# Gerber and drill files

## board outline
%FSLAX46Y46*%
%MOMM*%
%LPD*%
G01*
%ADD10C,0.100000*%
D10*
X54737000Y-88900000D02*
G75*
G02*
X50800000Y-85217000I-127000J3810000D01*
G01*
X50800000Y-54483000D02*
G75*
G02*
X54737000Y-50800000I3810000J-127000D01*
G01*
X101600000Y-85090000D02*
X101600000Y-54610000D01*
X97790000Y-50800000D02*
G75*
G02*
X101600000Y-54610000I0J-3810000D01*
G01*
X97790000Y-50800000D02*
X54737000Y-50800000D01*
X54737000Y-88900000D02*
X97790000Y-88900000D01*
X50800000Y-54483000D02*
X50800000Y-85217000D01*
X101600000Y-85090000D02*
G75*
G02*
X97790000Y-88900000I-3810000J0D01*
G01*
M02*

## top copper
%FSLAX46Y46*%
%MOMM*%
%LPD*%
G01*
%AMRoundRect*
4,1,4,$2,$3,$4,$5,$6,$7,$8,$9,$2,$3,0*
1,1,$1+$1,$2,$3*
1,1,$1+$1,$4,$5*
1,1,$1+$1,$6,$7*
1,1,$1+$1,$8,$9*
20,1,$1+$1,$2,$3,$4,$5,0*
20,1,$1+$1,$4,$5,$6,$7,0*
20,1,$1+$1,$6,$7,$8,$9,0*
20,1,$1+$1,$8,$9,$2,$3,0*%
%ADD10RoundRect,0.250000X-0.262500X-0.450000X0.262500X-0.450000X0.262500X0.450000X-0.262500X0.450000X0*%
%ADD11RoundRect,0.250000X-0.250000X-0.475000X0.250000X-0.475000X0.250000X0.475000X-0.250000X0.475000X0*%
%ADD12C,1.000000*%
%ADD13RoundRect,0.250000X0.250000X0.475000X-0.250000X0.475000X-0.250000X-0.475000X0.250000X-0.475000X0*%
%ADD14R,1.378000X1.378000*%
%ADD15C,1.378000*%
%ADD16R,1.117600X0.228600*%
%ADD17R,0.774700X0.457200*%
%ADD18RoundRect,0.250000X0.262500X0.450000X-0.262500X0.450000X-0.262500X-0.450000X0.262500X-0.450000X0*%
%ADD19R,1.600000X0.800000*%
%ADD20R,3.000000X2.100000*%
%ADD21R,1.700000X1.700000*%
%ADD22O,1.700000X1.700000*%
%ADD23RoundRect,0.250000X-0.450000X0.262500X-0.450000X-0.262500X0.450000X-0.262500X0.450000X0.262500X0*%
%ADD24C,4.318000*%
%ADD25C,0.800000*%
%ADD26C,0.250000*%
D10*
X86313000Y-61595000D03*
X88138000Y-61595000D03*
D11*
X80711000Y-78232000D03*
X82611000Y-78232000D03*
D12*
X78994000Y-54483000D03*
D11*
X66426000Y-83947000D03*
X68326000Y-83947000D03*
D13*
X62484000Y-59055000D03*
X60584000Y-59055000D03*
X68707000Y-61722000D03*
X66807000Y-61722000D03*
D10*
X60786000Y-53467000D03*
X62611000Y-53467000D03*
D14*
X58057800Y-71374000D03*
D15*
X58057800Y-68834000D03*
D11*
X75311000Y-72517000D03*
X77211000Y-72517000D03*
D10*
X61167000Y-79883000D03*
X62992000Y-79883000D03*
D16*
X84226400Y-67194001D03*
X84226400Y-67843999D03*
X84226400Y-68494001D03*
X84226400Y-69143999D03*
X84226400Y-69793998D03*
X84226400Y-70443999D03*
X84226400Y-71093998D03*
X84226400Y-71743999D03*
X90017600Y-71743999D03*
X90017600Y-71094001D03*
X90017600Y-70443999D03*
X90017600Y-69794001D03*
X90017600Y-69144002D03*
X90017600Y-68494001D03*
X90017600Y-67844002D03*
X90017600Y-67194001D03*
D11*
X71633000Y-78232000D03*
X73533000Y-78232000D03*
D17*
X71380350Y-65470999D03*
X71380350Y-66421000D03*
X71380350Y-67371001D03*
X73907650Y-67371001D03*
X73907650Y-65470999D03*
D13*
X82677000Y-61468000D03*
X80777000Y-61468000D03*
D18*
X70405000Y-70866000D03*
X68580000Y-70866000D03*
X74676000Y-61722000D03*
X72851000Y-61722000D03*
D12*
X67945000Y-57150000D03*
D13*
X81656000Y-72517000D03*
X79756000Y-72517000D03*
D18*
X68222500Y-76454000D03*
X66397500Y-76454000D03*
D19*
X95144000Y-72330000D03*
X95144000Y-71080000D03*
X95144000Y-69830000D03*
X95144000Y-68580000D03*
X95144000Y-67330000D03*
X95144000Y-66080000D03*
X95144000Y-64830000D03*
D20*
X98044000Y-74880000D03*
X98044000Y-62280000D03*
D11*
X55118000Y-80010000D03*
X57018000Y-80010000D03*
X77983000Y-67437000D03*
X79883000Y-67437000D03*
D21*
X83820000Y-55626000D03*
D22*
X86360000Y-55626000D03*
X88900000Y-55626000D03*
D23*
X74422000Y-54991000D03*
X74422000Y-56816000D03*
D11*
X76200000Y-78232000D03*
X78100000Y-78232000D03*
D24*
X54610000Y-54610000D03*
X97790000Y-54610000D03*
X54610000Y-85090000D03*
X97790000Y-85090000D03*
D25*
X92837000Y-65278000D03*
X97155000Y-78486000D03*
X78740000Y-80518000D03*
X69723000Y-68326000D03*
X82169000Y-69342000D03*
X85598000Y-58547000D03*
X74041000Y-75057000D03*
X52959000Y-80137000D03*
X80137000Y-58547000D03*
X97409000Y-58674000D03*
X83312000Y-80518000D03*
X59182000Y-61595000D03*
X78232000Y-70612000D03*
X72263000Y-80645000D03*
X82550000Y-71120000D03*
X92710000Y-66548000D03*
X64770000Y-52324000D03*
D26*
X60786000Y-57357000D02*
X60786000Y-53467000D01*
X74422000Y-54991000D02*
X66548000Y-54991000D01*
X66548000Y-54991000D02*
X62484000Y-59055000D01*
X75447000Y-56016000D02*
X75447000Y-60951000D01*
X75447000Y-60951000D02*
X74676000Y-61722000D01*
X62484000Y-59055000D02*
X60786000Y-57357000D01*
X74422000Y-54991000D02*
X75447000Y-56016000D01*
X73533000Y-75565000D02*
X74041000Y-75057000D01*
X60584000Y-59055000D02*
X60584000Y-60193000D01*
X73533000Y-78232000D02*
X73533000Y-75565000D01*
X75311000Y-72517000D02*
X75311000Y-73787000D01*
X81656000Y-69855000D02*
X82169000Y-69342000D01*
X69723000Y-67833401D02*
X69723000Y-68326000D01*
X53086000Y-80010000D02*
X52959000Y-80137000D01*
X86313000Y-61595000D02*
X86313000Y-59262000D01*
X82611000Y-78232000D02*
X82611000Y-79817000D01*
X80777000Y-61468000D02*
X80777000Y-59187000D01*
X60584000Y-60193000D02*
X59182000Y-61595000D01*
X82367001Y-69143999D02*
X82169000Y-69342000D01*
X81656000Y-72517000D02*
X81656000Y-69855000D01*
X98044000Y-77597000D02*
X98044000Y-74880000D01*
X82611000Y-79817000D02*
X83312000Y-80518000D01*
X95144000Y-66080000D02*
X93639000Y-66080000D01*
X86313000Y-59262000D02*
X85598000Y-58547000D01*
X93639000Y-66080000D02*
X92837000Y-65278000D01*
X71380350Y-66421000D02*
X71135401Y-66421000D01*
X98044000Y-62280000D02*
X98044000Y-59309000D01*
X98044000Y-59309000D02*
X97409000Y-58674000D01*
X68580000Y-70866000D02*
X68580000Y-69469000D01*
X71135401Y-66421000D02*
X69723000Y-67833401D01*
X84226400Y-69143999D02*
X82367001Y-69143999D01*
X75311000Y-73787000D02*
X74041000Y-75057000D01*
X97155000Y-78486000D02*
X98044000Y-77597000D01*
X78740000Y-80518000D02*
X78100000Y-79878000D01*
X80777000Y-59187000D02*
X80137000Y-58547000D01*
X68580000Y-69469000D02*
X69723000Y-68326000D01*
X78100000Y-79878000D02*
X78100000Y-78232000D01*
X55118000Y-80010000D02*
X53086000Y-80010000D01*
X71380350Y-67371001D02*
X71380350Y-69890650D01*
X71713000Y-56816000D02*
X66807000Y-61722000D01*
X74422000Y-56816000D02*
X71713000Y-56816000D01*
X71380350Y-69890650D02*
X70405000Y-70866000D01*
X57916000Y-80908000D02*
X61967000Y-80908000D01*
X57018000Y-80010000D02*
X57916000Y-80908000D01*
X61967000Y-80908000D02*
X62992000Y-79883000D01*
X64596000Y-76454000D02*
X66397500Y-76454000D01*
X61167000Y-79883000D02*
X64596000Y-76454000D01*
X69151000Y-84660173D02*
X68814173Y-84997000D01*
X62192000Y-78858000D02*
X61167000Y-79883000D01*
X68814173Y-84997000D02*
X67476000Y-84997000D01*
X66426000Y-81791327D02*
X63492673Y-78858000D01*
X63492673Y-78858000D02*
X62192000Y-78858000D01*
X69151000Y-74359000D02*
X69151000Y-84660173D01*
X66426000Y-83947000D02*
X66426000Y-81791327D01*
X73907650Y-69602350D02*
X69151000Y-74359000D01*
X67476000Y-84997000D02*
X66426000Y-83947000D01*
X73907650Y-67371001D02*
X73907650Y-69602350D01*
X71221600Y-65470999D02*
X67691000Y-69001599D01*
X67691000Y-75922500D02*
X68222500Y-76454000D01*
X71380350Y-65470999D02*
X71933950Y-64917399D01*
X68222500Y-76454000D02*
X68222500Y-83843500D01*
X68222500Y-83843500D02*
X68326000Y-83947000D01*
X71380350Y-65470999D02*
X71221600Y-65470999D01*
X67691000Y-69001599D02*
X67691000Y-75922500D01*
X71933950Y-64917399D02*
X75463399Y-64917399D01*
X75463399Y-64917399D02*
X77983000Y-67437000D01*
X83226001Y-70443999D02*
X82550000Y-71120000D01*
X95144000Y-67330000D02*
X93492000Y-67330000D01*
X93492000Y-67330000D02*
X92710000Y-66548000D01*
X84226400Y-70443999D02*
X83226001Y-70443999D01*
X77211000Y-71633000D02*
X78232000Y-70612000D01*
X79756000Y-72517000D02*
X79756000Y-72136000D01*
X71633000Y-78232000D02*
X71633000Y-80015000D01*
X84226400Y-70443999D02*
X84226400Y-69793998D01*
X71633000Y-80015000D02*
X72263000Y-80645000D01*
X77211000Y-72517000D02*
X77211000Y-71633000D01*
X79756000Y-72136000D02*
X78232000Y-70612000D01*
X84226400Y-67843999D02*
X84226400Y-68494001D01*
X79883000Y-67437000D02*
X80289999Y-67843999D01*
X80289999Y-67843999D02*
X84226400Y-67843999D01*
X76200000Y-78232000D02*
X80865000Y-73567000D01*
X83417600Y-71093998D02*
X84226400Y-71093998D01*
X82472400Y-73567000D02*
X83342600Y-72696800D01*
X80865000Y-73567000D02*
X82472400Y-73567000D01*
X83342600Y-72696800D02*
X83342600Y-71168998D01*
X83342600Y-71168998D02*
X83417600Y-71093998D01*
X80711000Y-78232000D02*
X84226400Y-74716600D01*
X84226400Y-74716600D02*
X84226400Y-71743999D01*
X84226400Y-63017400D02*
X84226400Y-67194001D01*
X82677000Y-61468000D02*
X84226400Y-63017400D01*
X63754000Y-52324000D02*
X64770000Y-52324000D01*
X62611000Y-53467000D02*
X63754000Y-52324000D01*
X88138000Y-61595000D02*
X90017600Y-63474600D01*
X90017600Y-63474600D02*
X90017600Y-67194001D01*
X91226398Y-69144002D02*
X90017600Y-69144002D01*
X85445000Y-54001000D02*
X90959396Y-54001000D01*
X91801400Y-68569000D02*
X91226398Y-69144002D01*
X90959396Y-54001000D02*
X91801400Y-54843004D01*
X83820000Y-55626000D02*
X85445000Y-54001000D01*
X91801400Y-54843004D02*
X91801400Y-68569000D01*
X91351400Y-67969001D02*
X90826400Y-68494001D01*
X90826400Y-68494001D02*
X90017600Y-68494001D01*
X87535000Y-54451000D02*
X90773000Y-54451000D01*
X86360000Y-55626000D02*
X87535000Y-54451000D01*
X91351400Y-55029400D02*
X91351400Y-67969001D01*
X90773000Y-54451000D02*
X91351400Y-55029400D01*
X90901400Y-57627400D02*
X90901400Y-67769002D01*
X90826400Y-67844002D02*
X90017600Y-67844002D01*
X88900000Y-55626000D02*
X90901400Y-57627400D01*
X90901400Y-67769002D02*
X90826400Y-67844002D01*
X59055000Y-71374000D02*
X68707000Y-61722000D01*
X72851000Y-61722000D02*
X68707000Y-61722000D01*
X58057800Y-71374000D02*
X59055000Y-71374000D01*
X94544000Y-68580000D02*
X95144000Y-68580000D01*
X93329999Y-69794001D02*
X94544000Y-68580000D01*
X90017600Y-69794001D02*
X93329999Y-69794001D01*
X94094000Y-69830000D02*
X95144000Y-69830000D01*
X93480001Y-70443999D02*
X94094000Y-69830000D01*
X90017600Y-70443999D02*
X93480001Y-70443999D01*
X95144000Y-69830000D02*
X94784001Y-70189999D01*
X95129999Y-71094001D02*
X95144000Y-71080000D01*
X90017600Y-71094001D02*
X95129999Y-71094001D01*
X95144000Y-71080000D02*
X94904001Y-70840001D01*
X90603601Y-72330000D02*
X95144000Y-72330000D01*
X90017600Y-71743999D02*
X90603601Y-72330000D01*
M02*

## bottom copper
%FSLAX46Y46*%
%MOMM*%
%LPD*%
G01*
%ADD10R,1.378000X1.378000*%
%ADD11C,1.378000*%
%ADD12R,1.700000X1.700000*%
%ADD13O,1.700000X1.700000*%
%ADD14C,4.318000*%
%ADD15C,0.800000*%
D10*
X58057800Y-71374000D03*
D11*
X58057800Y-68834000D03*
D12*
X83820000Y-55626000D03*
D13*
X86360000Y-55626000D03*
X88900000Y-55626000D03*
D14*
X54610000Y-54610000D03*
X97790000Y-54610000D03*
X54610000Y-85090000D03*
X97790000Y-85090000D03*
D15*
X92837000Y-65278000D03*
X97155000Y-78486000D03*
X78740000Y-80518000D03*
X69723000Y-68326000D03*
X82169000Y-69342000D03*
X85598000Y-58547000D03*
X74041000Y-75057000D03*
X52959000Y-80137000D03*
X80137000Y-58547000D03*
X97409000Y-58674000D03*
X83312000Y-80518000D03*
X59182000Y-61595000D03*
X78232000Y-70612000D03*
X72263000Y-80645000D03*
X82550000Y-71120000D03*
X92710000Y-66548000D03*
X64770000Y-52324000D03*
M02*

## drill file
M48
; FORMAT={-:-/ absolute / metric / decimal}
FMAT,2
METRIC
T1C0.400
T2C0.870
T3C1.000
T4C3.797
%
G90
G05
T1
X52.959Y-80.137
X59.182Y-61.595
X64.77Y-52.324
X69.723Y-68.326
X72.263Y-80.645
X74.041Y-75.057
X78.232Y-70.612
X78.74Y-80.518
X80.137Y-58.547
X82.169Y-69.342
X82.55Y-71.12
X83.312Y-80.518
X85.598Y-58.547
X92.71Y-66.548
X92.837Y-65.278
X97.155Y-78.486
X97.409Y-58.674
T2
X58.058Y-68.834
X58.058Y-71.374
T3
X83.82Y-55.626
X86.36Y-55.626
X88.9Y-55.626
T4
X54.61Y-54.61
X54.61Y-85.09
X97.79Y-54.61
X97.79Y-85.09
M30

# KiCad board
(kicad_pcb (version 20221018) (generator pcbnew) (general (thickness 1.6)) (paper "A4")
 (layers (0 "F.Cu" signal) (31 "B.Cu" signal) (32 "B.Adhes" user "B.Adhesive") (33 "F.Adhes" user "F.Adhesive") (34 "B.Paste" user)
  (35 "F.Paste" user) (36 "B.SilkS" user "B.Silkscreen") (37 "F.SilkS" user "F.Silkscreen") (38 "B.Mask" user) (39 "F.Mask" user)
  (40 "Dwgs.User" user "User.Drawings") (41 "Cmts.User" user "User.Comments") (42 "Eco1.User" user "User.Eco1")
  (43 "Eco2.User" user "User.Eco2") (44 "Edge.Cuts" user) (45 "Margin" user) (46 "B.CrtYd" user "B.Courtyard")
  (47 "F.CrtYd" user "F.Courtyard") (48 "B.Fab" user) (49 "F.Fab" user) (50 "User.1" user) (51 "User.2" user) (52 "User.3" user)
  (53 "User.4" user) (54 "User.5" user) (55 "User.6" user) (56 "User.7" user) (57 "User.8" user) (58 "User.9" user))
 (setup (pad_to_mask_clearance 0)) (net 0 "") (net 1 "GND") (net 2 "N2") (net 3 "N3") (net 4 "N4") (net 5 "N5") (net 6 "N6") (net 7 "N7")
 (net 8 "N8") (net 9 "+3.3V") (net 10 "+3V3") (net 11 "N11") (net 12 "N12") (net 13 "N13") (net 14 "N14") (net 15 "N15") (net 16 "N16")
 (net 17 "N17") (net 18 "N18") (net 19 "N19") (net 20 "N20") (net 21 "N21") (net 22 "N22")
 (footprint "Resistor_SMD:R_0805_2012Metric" (layer "F.Cu") (at 87.2255 61.595)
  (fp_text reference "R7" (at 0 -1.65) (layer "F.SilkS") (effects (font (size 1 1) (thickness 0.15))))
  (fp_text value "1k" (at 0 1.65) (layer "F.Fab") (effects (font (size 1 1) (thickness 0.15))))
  (pad "1" smd roundrect (at -0.9125 0) (size 1.025 1.4) (layers "F.Cu" "F.Paste" "F.Mask") (roundrect_rratio 0.243902) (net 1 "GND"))
  (pad "2" smd roundrect (at 0.9125 0) (size 1.025 1.4) (layers "F.Cu" "F.Paste" "F.Mask") (roundrect_rratio 0.243902) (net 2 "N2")))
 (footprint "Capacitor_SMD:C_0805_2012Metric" (layer "F.Cu") (at 81.661 78.232)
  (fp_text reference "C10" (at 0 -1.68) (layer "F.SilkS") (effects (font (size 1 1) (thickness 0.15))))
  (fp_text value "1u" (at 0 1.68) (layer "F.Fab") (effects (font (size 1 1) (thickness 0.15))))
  (pad "1" smd roundrect (at -0.95 0) (size 1 1.45) (layers "F.Cu" "F.Paste" "F.Mask") (roundrect_rratio 0.25) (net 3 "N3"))
  (pad "2" smd roundrect (at 0.95 0) (size 1 1.45) (layers "F.Cu" "F.Paste" "F.Mask") (roundrect_rratio 0.25) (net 1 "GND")))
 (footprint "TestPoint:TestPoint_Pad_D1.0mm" (layer "F.Cu") (at 78.994 54.483)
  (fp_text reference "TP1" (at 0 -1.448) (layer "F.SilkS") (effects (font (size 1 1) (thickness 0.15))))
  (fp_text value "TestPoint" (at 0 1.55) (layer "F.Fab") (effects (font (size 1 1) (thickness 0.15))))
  (pad "1" smd circle (at 0 0) (size 1 1) (layers "F.Cu" "F.Mask") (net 1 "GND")))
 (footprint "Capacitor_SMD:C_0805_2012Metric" (layer "F.Cu") (at 67.376 83.947)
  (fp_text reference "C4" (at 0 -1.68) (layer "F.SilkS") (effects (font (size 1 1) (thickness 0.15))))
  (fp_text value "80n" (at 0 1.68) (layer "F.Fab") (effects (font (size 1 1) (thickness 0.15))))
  (pad "1" smd roundrect (at -0.95 0) (size 1 1.45) (layers "F.Cu" "F.Paste" "F.Mask") (roundrect_rratio 0.25) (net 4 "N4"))
  (pad "2" smd roundrect (at 0.95 0) (size 1 1.45) (layers "F.Cu" "F.Paste" "F.Mask") (roundrect_rratio 0.25) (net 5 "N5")))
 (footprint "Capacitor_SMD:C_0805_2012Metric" (layer "F.Cu") (at 61.534 59.055 180)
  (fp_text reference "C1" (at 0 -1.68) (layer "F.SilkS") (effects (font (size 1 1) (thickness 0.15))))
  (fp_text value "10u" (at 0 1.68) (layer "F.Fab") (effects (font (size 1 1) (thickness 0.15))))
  (pad "1" smd roundrect (at -0.95 0 180) (size 1 1.45) (layers "F.Cu" "F.Paste" "F.Mask") (roundrect_rratio 0.25) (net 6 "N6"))
  (pad "2" smd roundrect (at 0.95 0 180) (size 1 1.45) (layers "F.Cu" "F.Paste" "F.Mask") (roundrect_rratio 0.25) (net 1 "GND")))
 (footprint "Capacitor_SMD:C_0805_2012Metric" (layer "F.Cu") (at 67.757 61.722 180)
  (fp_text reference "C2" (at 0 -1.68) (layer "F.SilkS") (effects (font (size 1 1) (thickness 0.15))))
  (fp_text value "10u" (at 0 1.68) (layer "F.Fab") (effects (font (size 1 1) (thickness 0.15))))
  (pad "1" smd roundrect (at -0.95 0 180) (size 1 1.45) (layers "F.Cu" "F.Paste" "F.Mask") (roundrect_rratio 0.25) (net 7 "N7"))
  (pad "2" smd roundrect (at 0.95 0 180) (size 1 1.45) (layers "F.Cu" "F.Paste" "F.Mask") (roundrect_rratio 0.25) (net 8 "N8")))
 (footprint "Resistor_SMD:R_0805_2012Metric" (layer "F.Cu") (at 61.6985 53.467)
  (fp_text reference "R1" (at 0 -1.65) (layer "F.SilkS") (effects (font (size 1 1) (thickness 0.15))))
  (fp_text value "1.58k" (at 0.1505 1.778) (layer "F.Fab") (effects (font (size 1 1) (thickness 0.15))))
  (pad "1" smd roundrect (at -0.9125 0) (size 1.025 1.4) (layers "F.Cu" "F.Paste" "F.Mask") (roundrect_rratio 0.243902) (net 6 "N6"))
  (pad "2" smd roundrect (at 0.9125 0) (size 1.025 1.4) (layers "F.Cu" "F.Paste" "F.Mask") (roundrect_rratio 0.243902) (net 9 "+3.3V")))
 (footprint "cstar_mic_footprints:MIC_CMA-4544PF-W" (layer "F.Cu") (at 56.0578 70.104)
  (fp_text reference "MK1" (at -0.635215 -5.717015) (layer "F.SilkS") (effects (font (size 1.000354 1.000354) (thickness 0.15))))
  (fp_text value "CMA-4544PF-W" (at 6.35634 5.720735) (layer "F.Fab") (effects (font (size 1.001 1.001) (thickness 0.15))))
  (pad "1" thru_hole rect (at 2 1.27) (size 1.378 1.378) (drill 0.87) (layers "*.Cu" "*.Mask") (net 7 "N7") (solder_mask_margin 0.102))
  (pad "2" thru_hole circle (at 2 -1.27) (size 1.378 1.378) (drill 0.87) (layers "*.Cu" "*.Mask") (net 1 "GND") (solder_mask_margin 0.102)))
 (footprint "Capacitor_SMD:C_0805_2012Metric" (layer "F.Cu") (at 76.261 72.517)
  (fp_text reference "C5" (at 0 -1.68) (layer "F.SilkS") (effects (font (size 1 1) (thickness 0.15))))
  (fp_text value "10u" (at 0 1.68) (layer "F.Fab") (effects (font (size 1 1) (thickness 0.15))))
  (pad "1" smd roundrect (at -0.95 0) (size 1 1.45) (layers "F.Cu" "F.Paste" "F.Mask") (roundrect_rratio 0.25) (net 1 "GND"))
  (pad "2" smd roundrect (at 0.95 0) (size 1 1.45) (layers "F.Cu" "F.Paste" "F.Mask") (roundrect_rratio 0.25) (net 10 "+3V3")))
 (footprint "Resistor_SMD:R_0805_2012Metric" (layer "F.Cu") (at 62.0795 79.883)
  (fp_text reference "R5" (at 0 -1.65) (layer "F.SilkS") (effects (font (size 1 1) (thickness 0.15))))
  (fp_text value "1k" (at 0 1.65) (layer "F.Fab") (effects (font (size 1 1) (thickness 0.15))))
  (pad "1" smd roundrect (at -0.9125 0) (size 1.025 1.4) (layers "F.Cu" "F.Paste" "F.Mask") (roundrect_rratio 0.243902) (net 4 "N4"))
  (pad "2" smd roundrect (at 0.9125 0) (size 1.025 1.4) (layers "F.Cu" "F.Paste" "F.Mask") (roundrect_rratio 0.243902) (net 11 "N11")))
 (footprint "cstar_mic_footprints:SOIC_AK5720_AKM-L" (layer "F.Cu") (at 87.122 69.469)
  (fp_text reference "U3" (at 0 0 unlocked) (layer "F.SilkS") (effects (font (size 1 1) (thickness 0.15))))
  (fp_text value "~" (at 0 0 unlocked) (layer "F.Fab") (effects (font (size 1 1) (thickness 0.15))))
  (pad "1" smd rect (at -2.8956 -2.274999) (size 1.1176 0.2286) (layers "F.Cu" "F.Paste" "F.Mask") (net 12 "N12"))
  (pad "2" smd rect (at -2.8956 -1.625001) (size 1.1176 0.2286) (layers "F.Cu" "F.Paste" "F.Mask") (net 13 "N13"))
  (pad "3" smd rect (at -2.8956 -0.974999) (size 1.1176 0.2286) (layers "F.Cu" "F.Paste" "F.Mask") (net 13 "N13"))
  (pad "4" smd rect (at -2.8956 -0.325001) (size 1.1176 0.2286) (layers "F.Cu" "F.Paste" "F.Mask") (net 1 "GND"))
  (pad "5" smd rect (at -2.8956 0.324998) (size 1.1176 0.2286) (layers "F.Cu" "F.Paste" "F.Mask") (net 10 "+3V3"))
  (pad "6" smd rect (at -2.8956 0.974999) (size 1.1176 0.2286) (layers "F.Cu" "F.Paste" "F.Mask") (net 10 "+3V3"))
  (pad "7" smd rect (at -2.8956 1.624998) (size 1.1176 0.2286) (layers "F.Cu" "F.Paste" "F.Mask") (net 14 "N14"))
  (pad "8" smd rect (at -2.8956 2.274999) (size 1.1176 0.2286) (layers "F.Cu" "F.Paste" "F.Mask") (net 3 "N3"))
  (pad "9" smd rect (at 2.8956 2.274999) (size 1.1176 0.2286) (layers "F.Cu" "F.Paste" "F.Mask") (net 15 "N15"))
  (pad "10" smd rect (at 2.8956 1.625001) (size 1.1176 0.2286) (layers "F.Cu" "F.Paste" "F.Mask") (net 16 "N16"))
  (pad "11" smd rect (at 2.8956 0.974999) (size 1.1176 0.2286) (layers "F.Cu" "F.Paste" "F.Mask") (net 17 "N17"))
  (pad "12" smd rect (at 2.8956 0.325001) (size 1.1176 0.2286) (layers "F.Cu" "F.Paste" "F.Mask") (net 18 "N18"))
  (pad "13" smd rect (at 2.8956 -0.324998) (size 1.1176 0.2286) (layers "F.Cu" "F.Paste" "F.Mask") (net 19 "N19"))
  (pad "14" smd rect (at 2.8956 -0.974999) (size 1.1176 0.2286) (layers "F.Cu" "F.Paste" "F.Mask") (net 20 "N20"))
  (pad "15" smd rect (at 2.8956 -1.624998) (size 1.1176 0.2286) (layers "F.Cu" "F.Paste" "F.Mask") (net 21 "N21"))
  (pad "16" smd rect (at 2.8956 -2.274999) (size 1.1176 0.2286) (layers "F.Cu" "F.Paste" "F.Mask") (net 2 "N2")))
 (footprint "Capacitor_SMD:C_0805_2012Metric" (layer "F.Cu") (at 72.583 78.232)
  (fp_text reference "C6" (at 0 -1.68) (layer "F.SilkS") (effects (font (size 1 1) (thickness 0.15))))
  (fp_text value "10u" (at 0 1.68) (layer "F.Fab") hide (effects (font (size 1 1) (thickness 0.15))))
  (pad "1" smd roundrect (at -0.95 0) (size 1 1.45) (layers "F.Cu" "F.Paste" "F.Mask") (roundrect_rratio 0.25) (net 10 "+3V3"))
  (pad "2" smd roundrect (at 0.95 0) (size 1 1.45) (layers "F.Cu" "F.Paste" "F.Mask") (roundrect_rratio 0.25) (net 1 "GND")))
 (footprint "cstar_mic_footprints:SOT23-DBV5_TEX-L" (layer "F.Cu") (at 72.644 66.421)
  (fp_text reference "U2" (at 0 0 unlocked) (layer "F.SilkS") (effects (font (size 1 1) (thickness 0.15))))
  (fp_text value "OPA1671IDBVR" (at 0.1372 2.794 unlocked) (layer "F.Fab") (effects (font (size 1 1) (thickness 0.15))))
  (pad "1" smd rect (at -1.26365 -0.950001) (size 0.7747 0.4572) (layers "F.Cu" "F.Paste" "F.Mask") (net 5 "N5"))
  (pad "2" smd rect (at -1.26365 0) (size 0.7747 0.4572) (layers "F.Cu" "F.Paste" "F.Mask") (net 1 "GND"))
  (pad "3" smd rect (at -1.26365 0.950001) (size 0.7747 0.4572) (layers "F.Cu" "F.Paste" "F.Mask") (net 8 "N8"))
  (pad "4" smd rect (at 1.26365 0.950001) (size 0.7747 0.4572) (layers "F.Cu" "F.Paste" "F.Mask") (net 4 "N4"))
  (pad "5" smd rect (at 1.26365 -0.950001) (size 0.7747 0.4572) (layers "F.Cu" "F.Paste" "F.Mask") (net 9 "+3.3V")))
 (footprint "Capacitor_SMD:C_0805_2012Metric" (layer "F.Cu") (at 81.727 61.468 180)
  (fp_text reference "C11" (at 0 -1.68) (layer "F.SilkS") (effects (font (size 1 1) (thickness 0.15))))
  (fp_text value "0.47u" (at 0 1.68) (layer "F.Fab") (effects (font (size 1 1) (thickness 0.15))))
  (pad "1" smd roundrect (at -0.95 0 180) (size 1 1.45) (layers "F.Cu" "F.Paste" "F.Mask") (roundrect_rratio 0.25) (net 12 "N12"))
  (pad "2" smd roundrect (at 0.95 0 180) (size 1 1.45) (layers "F.Cu" "F.Paste" "F.Mask") (roundrect_rratio 0.25) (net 1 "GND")))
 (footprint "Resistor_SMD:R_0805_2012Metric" (layer "F.Cu") (at 69.4925 70.866 180)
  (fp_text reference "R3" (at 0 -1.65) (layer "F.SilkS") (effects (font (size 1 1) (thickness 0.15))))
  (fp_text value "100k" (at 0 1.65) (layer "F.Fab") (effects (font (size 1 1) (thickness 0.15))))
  (pad "1" smd roundrect (at -0.9125 0 180) (size 1.025 1.4) (layers "F.Cu" "F.Paste" "F.Mask") (roundrect_rratio 0.243902) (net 8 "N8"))
  (pad "2" smd roundrect (at 0.9125 0 180) (size 1.025 1.4) (layers "F.Cu" "F.Paste" "F.Mask") (roundrect_rratio 0.243902) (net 1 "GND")))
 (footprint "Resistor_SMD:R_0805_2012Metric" (layer "F.Cu") (at 73.7635 61.722 180)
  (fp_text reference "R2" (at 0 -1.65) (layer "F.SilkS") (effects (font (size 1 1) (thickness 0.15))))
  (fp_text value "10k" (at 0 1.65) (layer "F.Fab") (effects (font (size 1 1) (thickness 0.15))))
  (pad "1" smd roundrect (at -0.9125 0 180) (size 1.025 1.4) (layers "F.Cu" "F.Paste" "F.Mask") (roundrect_rratio 0.243902) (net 6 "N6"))
  (pad "2" smd roundrect (at 0.9125 0 180) (size 1.025 1.4) (layers "F.Cu" "F.Paste" "F.Mask") (roundrect_rratio 0.243902) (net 7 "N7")))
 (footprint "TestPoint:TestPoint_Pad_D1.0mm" (layer "F.Cu") (at 67.945 57.15)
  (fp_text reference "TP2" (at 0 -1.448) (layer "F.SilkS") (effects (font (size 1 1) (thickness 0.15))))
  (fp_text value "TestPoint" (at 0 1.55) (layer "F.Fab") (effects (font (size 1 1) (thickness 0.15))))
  (pad "1" smd circle (at 0 0) (size 1 1) (layers "F.Cu" "F.Mask") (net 8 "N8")))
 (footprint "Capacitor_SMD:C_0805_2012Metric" (layer "F.Cu") (at 80.706 72.517 180)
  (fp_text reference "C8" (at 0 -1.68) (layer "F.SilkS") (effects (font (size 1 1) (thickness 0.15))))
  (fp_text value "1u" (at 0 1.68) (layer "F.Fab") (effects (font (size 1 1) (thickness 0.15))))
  (pad "1" smd roundrect (at -0.95 0 180) (size 1 1.45) (layers "F.Cu" "F.Paste" "F.Mask") (roundrect_rratio 0.25) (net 1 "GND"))
  (pad "2" smd roundrect (at 0.95 0 180) (size 1 1.45) (layers "F.Cu" "F.Paste" "F.Mask") (roundrect_rratio 0.25) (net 10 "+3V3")))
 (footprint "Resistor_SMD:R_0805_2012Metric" (layer "F.Cu") (at 67.31 76.454 180)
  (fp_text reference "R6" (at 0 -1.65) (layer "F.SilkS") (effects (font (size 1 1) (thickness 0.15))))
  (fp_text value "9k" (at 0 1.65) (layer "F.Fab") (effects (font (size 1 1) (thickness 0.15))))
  (pad "1" smd roundrect (at -0.9125 0 180) (size 1.025 1.4) (layers "F.Cu" "F.Paste" "F.Mask") (roundrect_rratio 0.243902) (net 5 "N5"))
  (pad "2" smd roundrect (at 0.9125 0 180) (size 1.025 1.4) (layers "F.Cu" "F.Paste" "F.Mask") (roundrect_rratio 0.243902) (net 4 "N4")))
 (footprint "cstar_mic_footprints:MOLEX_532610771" (layer "F.Cu") (at 97.544 68.58 90)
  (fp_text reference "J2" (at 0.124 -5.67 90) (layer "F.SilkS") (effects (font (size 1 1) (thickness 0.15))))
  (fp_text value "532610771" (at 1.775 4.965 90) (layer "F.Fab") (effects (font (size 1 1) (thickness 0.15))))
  (pad "1" smd rect (at -3.75 -2.4 90) (size 0.8 1.6) (layers "F.Cu" "F.Paste") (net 15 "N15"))
  (pad "2" smd rect (at -2.5 -2.4 90) (size 0.8 1.6) (layers "F.Cu" "F.Paste") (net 16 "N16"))
  (pad "3" smd rect (at -1.25 -2.4 90) (size 0.8 1.6) (layers "F.Cu" "F.Paste") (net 17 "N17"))
  (pad "4" smd rect (at 0 -2.4 90) (size 0.8 1.6) (layers "F.Cu" "F.Paste") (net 18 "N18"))
  (pad "5" smd rect (at 1.25 -2.4 90) (size 0.8 1.6) (layers "F.Cu" "F.Paste") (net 10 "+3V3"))
  (pad "6" smd rect (at 2.5 -2.4 90) (size 0.8 1.6) (layers "F.Cu" "F.Paste") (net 1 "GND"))
  (pad "7" smd rect (at 3.75 -2.4 90) (size 0.8 1.6) (layers "F.Cu" "F.Paste") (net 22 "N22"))
  (pad "S1" smd rect (at -6.3 0.5 90) (size 2.1 3) (layers "F.Cu" "F.Paste") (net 1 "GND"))
  (pad "S2" smd rect (at 6.3 0.5 90) (size 2.1 3) (layers "F.Cu" "F.Paste") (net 1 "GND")))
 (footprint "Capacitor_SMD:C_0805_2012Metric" (layer "F.Cu") (at 56.068 80.01)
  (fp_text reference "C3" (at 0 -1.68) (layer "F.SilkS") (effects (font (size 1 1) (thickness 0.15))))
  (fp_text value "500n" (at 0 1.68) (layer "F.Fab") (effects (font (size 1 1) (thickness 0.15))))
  (pad "1" smd roundrect (at -0.95 0) (size 1 1.45) (layers "F.Cu" "F.Paste" "F.Mask") (roundrect_rratio 0.25) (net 1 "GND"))
  (pad "2" smd roundrect (at 0.95 0) (size 1 1.45) (layers "F.Cu" "F.Paste" "F.Mask") (roundrect_rratio 0.25) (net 11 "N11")))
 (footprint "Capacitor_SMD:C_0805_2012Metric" (layer "F.Cu") (at 78.933 67.437)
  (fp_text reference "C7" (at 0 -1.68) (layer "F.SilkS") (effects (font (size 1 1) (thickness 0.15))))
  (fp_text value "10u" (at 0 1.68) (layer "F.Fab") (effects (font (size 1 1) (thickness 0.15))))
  (pad "1" smd roundrect (at -0.95 0) (size 1 1.45) (layers "F.Cu" "F.Paste" "F.Mask") (roundrect_rratio 0.25) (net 5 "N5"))
  (pad "2" smd roundrect (at 0.95 0) (size 1 1.45) (layers "F.Cu" "F.Paste" "F.Mask") (roundrect_rratio 0.25) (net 13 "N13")))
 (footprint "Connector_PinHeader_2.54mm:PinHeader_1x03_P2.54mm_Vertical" (layer "F.Cu") (at 83.82 55.626 90)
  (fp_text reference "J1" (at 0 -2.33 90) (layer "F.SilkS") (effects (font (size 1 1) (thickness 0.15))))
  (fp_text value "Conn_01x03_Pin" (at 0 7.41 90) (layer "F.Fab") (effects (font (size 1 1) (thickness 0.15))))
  (pad "1" thru_hole rect (at 0 0 90) (size 1.7 1.7) (drill 1) (layers "*.Cu" "*.Mask") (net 19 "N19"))
  (pad "2" thru_hole oval (at 0 2.54 90) (size 1.7 1.7) (drill 1) (layers "*.Cu" "*.Mask") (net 20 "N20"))
  (pad "3" thru_hole oval (at 0 5.08 90) (size 1.7 1.7) (drill 1) (layers "*.Cu" "*.Mask") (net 21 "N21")))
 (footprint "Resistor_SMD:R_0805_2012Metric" (layer "F.Cu") (at 74.422 55.9035 -90)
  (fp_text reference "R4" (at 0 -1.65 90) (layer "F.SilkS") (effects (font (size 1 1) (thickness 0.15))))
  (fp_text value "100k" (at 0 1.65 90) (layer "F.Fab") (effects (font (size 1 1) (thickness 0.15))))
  (pad "1" smd roundrect (at -0.9125 0 270) (size 1.025 1.4) (layers "F.Cu" "F.Paste" "F.Mask") (roundrect_rratio 0.243902) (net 6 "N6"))
  (pad "2" smd roundrect (at 0.9125 0 270) (size 1.025 1.4) (layers "F.Cu" "F.Paste" "F.Mask") (roundrect_rratio 0.243902) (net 8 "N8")))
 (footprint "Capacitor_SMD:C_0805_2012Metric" (layer "F.Cu") (at 77.15 78.232)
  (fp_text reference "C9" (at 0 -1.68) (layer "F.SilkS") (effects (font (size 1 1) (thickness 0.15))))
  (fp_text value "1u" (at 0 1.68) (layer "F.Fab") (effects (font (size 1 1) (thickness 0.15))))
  (pad "1" smd roundrect (at -0.95 0) (size 1 1.45) (layers "F.Cu" "F.Paste" "F.Mask") (roundrect_rratio 0.25) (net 14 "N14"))
  (pad "2" smd roundrect (at 0.95 0) (size 1 1.45) (layers "F.Cu" "F.Paste" "F.Mask") (roundrect_rratio 0.25) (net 1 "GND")))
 (gr_arc (start 54.737 88.9) (mid 52.005726 87.873879) (end 50.8 85.217) (stroke (width 0.1) (type default)) (layer "Edge.Cuts"))
 (gr_arc (start 50.8 54.483) (mid 52.005726 51.826121) (end 54.737 50.8) (stroke (width 0.1) (type default)) (layer "Edge.Cuts"))
 (gr_line (start 101.6 85.09) (end 101.6 54.61) (stroke (width 0.1) (type default)) (layer "Edge.Cuts"))
 (gr_arc (start 97.79 50.8) (mid 100.484076 51.915923) (end 101.6 54.61) (stroke (width 0.1) (type default)) (layer "Edge.Cuts"))
 (gr_line (start 97.79 50.8) (end 54.737 50.8) (stroke (width 0.1) (type default)) (layer "Edge.Cuts"))
 (gr_line (start 54.737 88.9) (end 97.79 88.9) (stroke (width 0.1) (type default)) (layer "Edge.Cuts"))
 (gr_line (start 50.8 54.483) (end 50.8 85.217) (stroke (width 0.1) (type default)) (layer "Edge.Cuts"))
 (gr_arc (start 101.6 85.09) (mid 100.484077 87.784077) (end 97.79 88.9) (stroke (width 0.1) (type default)) (layer "Edge.Cuts"))
 (via (at 54.61 54.61) (size 4.318) (drill 3.7973) (layers "F.Cu" "B.Cu") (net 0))
 (via (at 97.79 54.61) (size 4.318) (drill 3.7973) (layers "F.Cu" "B.Cu") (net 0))
 (via (at 54.61 85.09) (size 4.318) (drill 3.7973) (layers "F.Cu" "B.Cu") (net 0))
 (via (at 97.79 85.09) (size 4.318) (drill 3.7973) (layers "F.Cu" "B.Cu") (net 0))
 (segment (start 60.786 57.357) (end 60.786 53.467) (width 0.25) (layer "F.Cu") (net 6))
 (segment (start 74.422 54.991) (end 66.548 54.991) (width 0.25) (layer "F.Cu") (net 6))
 (segment (start 66.548 54.991) (end 62.484 59.055) (width 0.25) (layer "F.Cu") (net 6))
 (segment (start 75.447 56.016) (end 75.447 60.951) (width 0.25) (layer "F.Cu") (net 6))
 (segment (start 75.447 60.951) (end 74.676 61.722) (width 0.25) (layer "F.Cu") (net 6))
 (segment (start 62.484 59.055) (end 60.786 57.357) (width 0.25) (layer "F.Cu") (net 6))
 (segment (start 74.422 54.991) (end 75.447 56.016) (width 0.25) (layer "F.Cu") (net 6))
 (segment (start 73.533 75.565) (end 74.041 75.057) (width 0.25) (layer "F.Cu") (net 1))
 (segment (start 60.584 59.055) (end 60.584 60.193) (width 0.25) (layer "F.Cu") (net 1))
 (segment (start 73.533 78.232) (end 73.533 75.565) (width 0.25) (layer "F.Cu") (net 1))
 (segment (start 75.311 72.517) (end 75.311 73.787) (width 0.25) (layer "F.Cu") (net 1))
 (segment (start 81.656 69.855) (end 82.169 69.342) (width 0.25) (layer "F.Cu") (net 1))
 (segment (start 69.723 67.833401) (end 69.723 68.326) (width 0.25) (layer "F.Cu") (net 1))
 (segment (start 53.086 80.01) (end 52.959 80.137) (width 0.25) (layer "F.Cu") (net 1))
 (segment (start 86.313 61.595) (end 86.313 59.262) (width 0.25) (layer "F.Cu") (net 1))
 (segment (start 82.611 78.232) (end 82.611 79.817) (width 0.25) (layer "F.Cu") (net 1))
 (segment (start 80.777 61.468) (end 80.777 59.187) (width 0.25) (layer "F.Cu") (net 1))
 (segment (start 60.584 60.193) (end 59.182 61.595) (width 0.25) (layer "F.Cu") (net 1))
 (segment (start 82.367001 69.143999) (end 82.169 69.342) (width 0.25) (layer "F.Cu") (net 1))
 (segment (start 81.656 72.517) (end 81.656 69.855) (width 0.25) (layer "F.Cu") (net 1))
 (segment (start 98.044 77.597) (end 98.044 74.88) (width 0.25) (layer "F.Cu") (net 1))
 (segment (start 82.611 79.817) (end 83.312 80.518) (width 0.25) (layer "F.Cu") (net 1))
 (segment (start 95.144 66.08) (end 93.639 66.08) (width 0.25) (layer "F.Cu") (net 1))
 (segment (start 86.313 59.262) (end 85.598 58.547) (width 0.25) (layer "F.Cu") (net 1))
 (segment (start 93.639 66.08) (end 92.837 65.278) (width 0.25) (layer "F.Cu") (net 1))
 (segment (start 71.38035 66.421) (end 71.135401 66.421) (width 0.25) (layer "F.Cu") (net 1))
 (segment (start 98.044 62.28) (end 98.044 59.309) (width 0.25) (layer "F.Cu") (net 1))
 (segment (start 98.044 59.309) (end 97.409 58.674) (width 0.25) (layer "F.Cu") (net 1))
 (segment (start 68.58 70.866) (end 68.58 69.469) (width 0.25) (layer "F.Cu") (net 1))
 (segment (start 71.135401 66.421) (end 69.723 67.833401) (width 0.25) (layer "F.Cu") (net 1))
 (segment (start 84.2264 69.143999) (end 82.367001 69.143999) (width 0.25) (layer "F.Cu") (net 1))
 (segment (start 75.311 73.787) (end 74.041 75.057) (width 0.25) (layer "F.Cu") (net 1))
 (segment (start 97.155 78.486) (end 98.044 77.597) (width 0.25) (layer "F.Cu") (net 1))
 (segment (start 78.74 80.518) (end 78.1 79.878) (width 0.25) (layer "F.Cu") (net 1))
 (segment (start 80.777 59.187) (end 80.137 58.547) (width 0.25) (layer "F.Cu") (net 1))
 (segment (start 68.58 69.469) (end 69.723 68.326) (width 0.25) (layer "F.Cu") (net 1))
 (segment (start 78.1 79.878) (end 78.1 78.232) (width 0.25) (layer "F.Cu") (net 1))
 (segment (start 55.118 80.01) (end 53.086 80.01) (width 0.25) (layer "F.Cu") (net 1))
 (via (at 92.837 65.278) (size 0.8) (drill 0.4) (layers "F.Cu" "B.Cu") (free) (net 1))
 (via (at 97.155 78.486) (size 0.8) (drill 0.4) (layers "F.Cu" "B.Cu") (free) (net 1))
 (via (at 78.74 80.518) (size 0.8) (drill 0.4) (layers "F.Cu" "B.Cu") (free) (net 1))
 (via (at 69.723 68.326) (size 0.8) (drill 0.4) (layers "F.Cu" "B.Cu") (free) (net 1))
 (via (at 82.169 69.342) (size 0.8) (drill 0.4) (layers "F.Cu" "B.Cu") (free) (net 1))
 (via (at 85.598 58.547) (size 0.8) (drill 0.4) (layers "F.Cu" "B.Cu") (free) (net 1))
 (via (at 74.041 75.057) (size 0.8) (drill 0.4) (layers "F.Cu" "B.Cu") (free) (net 1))
 (via (at 52.959 80.137) (size 0.8) (drill 0.4) (layers "F.Cu" "B.Cu") (free) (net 1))
 (via (at 80.137 58.547) (size 0.8) (drill 0.4) (layers "F.Cu" "B.Cu") (free) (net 1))
 (via (at 97.409 58.674) (size 0.8) (drill 0.4) (layers "F.Cu" "B.Cu") (free) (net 1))
 (via (at 83.312 80.518) (size 0.8) (drill 0.4) (layers "F.Cu" "B.Cu") (free) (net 1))
 (via (at 59.182 61.595) (size 0.8) (drill 0.4) (layers "F.Cu" "B.Cu") (free) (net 1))
 (segment (start 71.38035 67.371001) (end 71.38035 69.89065) (width 0.25) (layer "F.Cu") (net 8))
 (segment (start 71.713 56.816) (end 66.807 61.722) (width 0.25) (layer "F.Cu") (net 8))
 (segment (start 74.422 56.816) (end 71.713 56.816) (width 0.25) (layer "F.Cu") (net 8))
 (segment (start 71.38035 69.89065) (end 70.405 70.866) (width 0.25) (layer "F.Cu") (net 8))
 (segment (start 57.916 80.908) (end 61.967 80.908) (width 0.25) (layer "F.Cu") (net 11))
 (segment (start 57.018 80.01) (end 57.916 80.908) (width 0.25) (layer "F.Cu") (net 11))
 (segment (start 61.967 80.908) (end 62.992 79.883) (width 0.25) (layer "F.Cu") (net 11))
 (segment (start 64.596 76.454) (end 66.3975 76.454) (width 0.25) (layer "F.Cu") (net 4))
 (segment (start 61.167 79.883) (end 64.596 76.454) (width 0.25) (layer "F.Cu") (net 4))
 (segment (start 69.151 84.660173) (end 68.814173 84.997) (width 0.25) (layer "F.Cu") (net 4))
 (segment (start 62.192 78.858) (end 61.167 79.883) (width 0.25) (layer "F.Cu") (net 4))
 (segment (start 68.814173 84.997) (end 67.476 84.997) (width 0.25) (layer "F.Cu") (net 4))
 (segment (start 66.426 81.791327) (end 63.492673 78.858) (width 0.25) (layer "F.Cu") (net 4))
 (segment (start 63.492673 78.858) (end 62.192 78.858) (width 0.25) (layer "F.Cu") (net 4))
 (segment (start 69.151 74.359) (end 69.151 84.660173) (width 0.25) (layer "F.Cu") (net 4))
 (segment (start 66.426 83.947) (end 66.426 81.791327) (width 0.25) (layer "F.Cu") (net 4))
 (segment (start 73.90765 69.60235) (end 69.151 74.359) (width 0.25) (layer "F.Cu") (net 4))
 (segment (start 67.476 84.997) (end 66.426 83.947) (width 0.25) (layer "F.Cu") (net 4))
 (segment (start 73.90765 67.371001) (end 73.90765 69.60235) (width 0.25) (layer "F.Cu") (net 4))
 (segment (start 71.2216 65.470999) (end 67.691 69.001599) (width 0.25) (layer "F.Cu") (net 5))
 (segment (start 67.691 75.9225) (end 68.2225 76.454) (width 0.25) (layer "F.Cu") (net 5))
 (segment (start 71.38035 65.470999) (end 71.93395 64.917399) (width 0.25) (layer "F.Cu") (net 5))
 (segment (start 68.2225 76.454) (end 68.2225 83.8435) (width 0.25) (layer "F.Cu") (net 5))
 (segment (start 68.2225 83.8435) (end 68.326 83.947) (width 0.25) (layer "F.Cu") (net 5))
 (segment (start 71.38035 65.470999) (end 71.2216 65.470999) (width 0.25) (layer "F.Cu") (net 5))
 (segment (start 67.691 69.001599) (end 67.691 75.9225) (width 0.25) (layer "F.Cu") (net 5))
 (segment (start 71.93395 64.917399) (end 75.463399 64.917399) (width 0.25) (layer "F.Cu") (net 5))
 (segment (start 75.463399 64.917399) (end 77.983 67.437) (width 0.25) (layer "F.Cu") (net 5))
 (segment (start 83.226001 70.443999) (end 82.55 71.12) (width 0.25) (layer "F.Cu") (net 10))
 (segment (start 95.144 67.33) (end 93.492 67.33) (width 0.25) (layer "F.Cu") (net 10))
 (segment (start 93.492 67.33) (end 92.71 66.548) (width 0.25) (layer "F.Cu") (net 10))
 (segment (start 84.2264 70.443999) (end 83.226001 70.443999) (width 0.25) (layer "F.Cu") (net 10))
 (segment (start 77.211 71.633) (end 78.232 70.612) (width 0.25) (layer "F.Cu") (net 10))
 (segment (start 79.756 72.517) (end 79.756 72.136) (width 0.25) (layer "F.Cu") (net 10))
 (segment (start 71.633 78.232) (end 71.633 80.015) (width 0.25) (layer "F.Cu") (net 10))
 (segment (start 84.2264 70.443999) (end 84.2264 69.793998) (width 0.25) (layer "F.Cu") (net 10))
 (segment (start 71.633 80.015) (end 72.263 80.645) (width 0.25) (layer "F.Cu") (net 10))
 (segment (start 77.211 72.517) (end 77.211 71.633) (width 0.25) (layer "F.Cu") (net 10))
 (segment (start 79.756 72.136) (end 78.232 70.612) (width 0.25) (layer "F.Cu") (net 10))
 (via (at 78.232 70.612) (size 0.8) (drill 0.4) (layers "F.Cu" "B.Cu") (free) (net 10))
 (via (at 72.263 80.645) (size 0.8) (drill 0.4) (layers "F.Cu" "B.Cu") (free) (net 10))
 (via (at 82.55 71.12) (size 0.8) (drill 0.4) (layers "F.Cu" "B.Cu") (free) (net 10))
 (via (at 92.71 66.548) (size 0.8) (drill 0.4) (layers "F.Cu" "B.Cu") (free) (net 10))
 (segment (start 84.2264 67.843999) (end 84.2264 68.494001) (width 0.25) (layer "F.Cu") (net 13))
 (segment (start 79.883 67.437) (end 80.289999 67.843999) (width 0.25) (layer "F.Cu") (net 13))
 (segment (start 80.289999 67.843999) (end 84.2264 67.843999) (width 0.25) (layer "F.Cu") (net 13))
 (segment (start 76.2 78.232) (end 80.865 73.567) (width 0.25) (layer "F.Cu") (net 14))
 (segment (start 83.4176 71.093998) (end 84.2264 71.093998) (width 0.25) (layer "F.Cu") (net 14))
 (segment (start 82.4724 73.567) (end 83.3426 72.6968) (width 0.25) (layer "F.Cu") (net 14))
 (segment (start 80.865 73.567) (end 82.4724 73.567) (width 0.25) (layer "F.Cu") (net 14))
 (segment (start 83.3426 72.6968) (end 83.3426 71.168998) (width 0.25) (layer "F.Cu") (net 14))
 (segment (start 83.3426 71.168998) (end 83.4176 71.093998) (width 0.25) (layer "F.Cu") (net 14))
 (segment (start 80.711 78.232) (end 84.2264 74.7166) (width 0.25) (layer "F.Cu") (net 3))
 (segment (start 84.2264 74.7166) (end 84.2264 71.743999) (width 0.25) (layer "F.Cu") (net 3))
 (segment (start 84.2264 63.0174) (end 84.2264 67.194001) (width 0.25) (layer "F.Cu") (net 12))
 (segment (start 82.677 61.468) (end 84.2264 63.0174) (width 0.25) (layer "F.Cu") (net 12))
 (segment (start 63.754 52.324) (end 64.77 52.324) (width 0.25) (layer "F.Cu") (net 9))
 (segment (start 62.611 53.467) (end 63.754 52.324) (width 0.25) (layer "F.Cu") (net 9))
 (via (at 64.77 52.324) (size 0.8) (drill 0.4) (layers "F.Cu" "B.Cu") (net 9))
 (segment (start 88.138 61.595) (end 90.0176 63.4746) (width 0.25) (layer "F.Cu") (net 2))
 (segment (start 90.0176 63.4746) (end 90.0176 67.194001) (width 0.25) (layer "F.Cu") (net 2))
 (segment (start 91.226398 69.144002) (end 90.0176 69.144002) (width 0.25) (layer "F.Cu") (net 19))
 (segment (start 85.445 54.001) (end 90.959396 54.001) (width 0.25) (layer "F.Cu") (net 19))
 (segment (start 91.8014 68.569) (end 91.226398 69.144002) (width 0.25) (layer "F.Cu") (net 19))
 (segment (start 90.959396 54.001) (end 91.8014 54.843004) (width 0.25) (layer "F.Cu") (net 19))
 (segment (start 83.82 55.626) (end 85.445 54.001) (width 0.25) (layer "F.Cu") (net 19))
 (segment (start 91.8014 54.843004) (end 91.8014 68.569) (width 0.25) (layer "F.Cu") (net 19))
 (segment (start 91.3514 67.969001) (end 90.8264 68.494001) (width 0.25) (layer "F.Cu") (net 20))
 (segment (start 90.8264 68.494001) (end 90.0176 68.494001) (width 0.25) (layer "F.Cu") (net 20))
 (segment (start 87.535 54.451) (end 90.773 54.451) (width 0.25) (layer "F.Cu") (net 20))
 (segment (start 86.36 55.626) (end 87.535 54.451) (width 0.25) (layer "F.Cu") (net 20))
 (segment (start 91.3514 55.0294) (end 91.3514 67.969001) (width 0.25) (layer "F.Cu") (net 20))
 (segment (start 90.773 54.451) (end 91.3514 55.0294) (width 0.25) (layer "F.Cu") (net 20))
 (segment (start 90.9014 57.6274) (end 90.9014 67.769002) (width 0.25) (layer "F.Cu") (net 21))
 (segment (start 90.8264 67.844002) (end 90.0176 67.844002) (width 0.25) (layer "F.Cu") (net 21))
 (segment (start 88.9 55.626) (end 90.9014 57.6274) (width 0.25) (layer "F.Cu") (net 21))
 (segment (start 90.9014 67.769002) (end 90.8264 67.844002) (width 0.25) (layer "F.Cu") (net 21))
 (segment (start 59.055 71.374) (end 68.707 61.722) (width 0.25) (layer "F.Cu") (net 7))
 (segment (start 72.851 61.722) (end 68.707 61.722) (width 0.25) (layer "F.Cu") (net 7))
 (segment (start 58.0578 71.374) (end 59.055 71.374) (width 0.25) (layer "F.Cu") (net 7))
 (segment (start 94.544 68.58) (end 95.144 68.58) (width 0.25) (layer "F.Cu") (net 18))
 (segment (start 93.329999 69.794001) (end 94.544 68.58) (width 0.25) (layer "F.Cu") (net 18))
 (segment (start 90.0176 69.794001) (end 93.329999 69.794001) (width 0.25) (layer "F.Cu") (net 18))
 (segment (start 94.094 69.83) (end 95.144 69.83) (width 0.25) (layer "F.Cu") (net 17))
 (segment (start 93.480001 70.443999) (end 94.094 69.83) (width 0.25) (layer "F.Cu") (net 17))
 (segment (start 90.0176 70.443999) (end 93.480001 70.443999) (width 0.25) (layer "F.Cu") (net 17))
 (segment (start 95.144 69.83) (end 94.784001 70.189999) (width 0.25) (layer "F.Cu") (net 17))
 (segment (start 95.129999 71.094001) (end 95.144 71.08) (width 0.25) (layer "F.Cu") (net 16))
 (segment (start 90.0176 71.094001) (end 95.129999 71.094001) (width 0.25) (layer "F.Cu") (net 16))
 (segment (start 95.144 71.08) (end 94.904001 70.840001) (width 0.25) (layer "F.Cu") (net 16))
 (segment (start 90.603601 72.33) (end 95.144 72.33) (width 0.25) (layer "F.Cu") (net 15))
 (segment (start 90.0176 71.743999) (end 90.603601 72.33) (width 0.25) (layer "F.Cu") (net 15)))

